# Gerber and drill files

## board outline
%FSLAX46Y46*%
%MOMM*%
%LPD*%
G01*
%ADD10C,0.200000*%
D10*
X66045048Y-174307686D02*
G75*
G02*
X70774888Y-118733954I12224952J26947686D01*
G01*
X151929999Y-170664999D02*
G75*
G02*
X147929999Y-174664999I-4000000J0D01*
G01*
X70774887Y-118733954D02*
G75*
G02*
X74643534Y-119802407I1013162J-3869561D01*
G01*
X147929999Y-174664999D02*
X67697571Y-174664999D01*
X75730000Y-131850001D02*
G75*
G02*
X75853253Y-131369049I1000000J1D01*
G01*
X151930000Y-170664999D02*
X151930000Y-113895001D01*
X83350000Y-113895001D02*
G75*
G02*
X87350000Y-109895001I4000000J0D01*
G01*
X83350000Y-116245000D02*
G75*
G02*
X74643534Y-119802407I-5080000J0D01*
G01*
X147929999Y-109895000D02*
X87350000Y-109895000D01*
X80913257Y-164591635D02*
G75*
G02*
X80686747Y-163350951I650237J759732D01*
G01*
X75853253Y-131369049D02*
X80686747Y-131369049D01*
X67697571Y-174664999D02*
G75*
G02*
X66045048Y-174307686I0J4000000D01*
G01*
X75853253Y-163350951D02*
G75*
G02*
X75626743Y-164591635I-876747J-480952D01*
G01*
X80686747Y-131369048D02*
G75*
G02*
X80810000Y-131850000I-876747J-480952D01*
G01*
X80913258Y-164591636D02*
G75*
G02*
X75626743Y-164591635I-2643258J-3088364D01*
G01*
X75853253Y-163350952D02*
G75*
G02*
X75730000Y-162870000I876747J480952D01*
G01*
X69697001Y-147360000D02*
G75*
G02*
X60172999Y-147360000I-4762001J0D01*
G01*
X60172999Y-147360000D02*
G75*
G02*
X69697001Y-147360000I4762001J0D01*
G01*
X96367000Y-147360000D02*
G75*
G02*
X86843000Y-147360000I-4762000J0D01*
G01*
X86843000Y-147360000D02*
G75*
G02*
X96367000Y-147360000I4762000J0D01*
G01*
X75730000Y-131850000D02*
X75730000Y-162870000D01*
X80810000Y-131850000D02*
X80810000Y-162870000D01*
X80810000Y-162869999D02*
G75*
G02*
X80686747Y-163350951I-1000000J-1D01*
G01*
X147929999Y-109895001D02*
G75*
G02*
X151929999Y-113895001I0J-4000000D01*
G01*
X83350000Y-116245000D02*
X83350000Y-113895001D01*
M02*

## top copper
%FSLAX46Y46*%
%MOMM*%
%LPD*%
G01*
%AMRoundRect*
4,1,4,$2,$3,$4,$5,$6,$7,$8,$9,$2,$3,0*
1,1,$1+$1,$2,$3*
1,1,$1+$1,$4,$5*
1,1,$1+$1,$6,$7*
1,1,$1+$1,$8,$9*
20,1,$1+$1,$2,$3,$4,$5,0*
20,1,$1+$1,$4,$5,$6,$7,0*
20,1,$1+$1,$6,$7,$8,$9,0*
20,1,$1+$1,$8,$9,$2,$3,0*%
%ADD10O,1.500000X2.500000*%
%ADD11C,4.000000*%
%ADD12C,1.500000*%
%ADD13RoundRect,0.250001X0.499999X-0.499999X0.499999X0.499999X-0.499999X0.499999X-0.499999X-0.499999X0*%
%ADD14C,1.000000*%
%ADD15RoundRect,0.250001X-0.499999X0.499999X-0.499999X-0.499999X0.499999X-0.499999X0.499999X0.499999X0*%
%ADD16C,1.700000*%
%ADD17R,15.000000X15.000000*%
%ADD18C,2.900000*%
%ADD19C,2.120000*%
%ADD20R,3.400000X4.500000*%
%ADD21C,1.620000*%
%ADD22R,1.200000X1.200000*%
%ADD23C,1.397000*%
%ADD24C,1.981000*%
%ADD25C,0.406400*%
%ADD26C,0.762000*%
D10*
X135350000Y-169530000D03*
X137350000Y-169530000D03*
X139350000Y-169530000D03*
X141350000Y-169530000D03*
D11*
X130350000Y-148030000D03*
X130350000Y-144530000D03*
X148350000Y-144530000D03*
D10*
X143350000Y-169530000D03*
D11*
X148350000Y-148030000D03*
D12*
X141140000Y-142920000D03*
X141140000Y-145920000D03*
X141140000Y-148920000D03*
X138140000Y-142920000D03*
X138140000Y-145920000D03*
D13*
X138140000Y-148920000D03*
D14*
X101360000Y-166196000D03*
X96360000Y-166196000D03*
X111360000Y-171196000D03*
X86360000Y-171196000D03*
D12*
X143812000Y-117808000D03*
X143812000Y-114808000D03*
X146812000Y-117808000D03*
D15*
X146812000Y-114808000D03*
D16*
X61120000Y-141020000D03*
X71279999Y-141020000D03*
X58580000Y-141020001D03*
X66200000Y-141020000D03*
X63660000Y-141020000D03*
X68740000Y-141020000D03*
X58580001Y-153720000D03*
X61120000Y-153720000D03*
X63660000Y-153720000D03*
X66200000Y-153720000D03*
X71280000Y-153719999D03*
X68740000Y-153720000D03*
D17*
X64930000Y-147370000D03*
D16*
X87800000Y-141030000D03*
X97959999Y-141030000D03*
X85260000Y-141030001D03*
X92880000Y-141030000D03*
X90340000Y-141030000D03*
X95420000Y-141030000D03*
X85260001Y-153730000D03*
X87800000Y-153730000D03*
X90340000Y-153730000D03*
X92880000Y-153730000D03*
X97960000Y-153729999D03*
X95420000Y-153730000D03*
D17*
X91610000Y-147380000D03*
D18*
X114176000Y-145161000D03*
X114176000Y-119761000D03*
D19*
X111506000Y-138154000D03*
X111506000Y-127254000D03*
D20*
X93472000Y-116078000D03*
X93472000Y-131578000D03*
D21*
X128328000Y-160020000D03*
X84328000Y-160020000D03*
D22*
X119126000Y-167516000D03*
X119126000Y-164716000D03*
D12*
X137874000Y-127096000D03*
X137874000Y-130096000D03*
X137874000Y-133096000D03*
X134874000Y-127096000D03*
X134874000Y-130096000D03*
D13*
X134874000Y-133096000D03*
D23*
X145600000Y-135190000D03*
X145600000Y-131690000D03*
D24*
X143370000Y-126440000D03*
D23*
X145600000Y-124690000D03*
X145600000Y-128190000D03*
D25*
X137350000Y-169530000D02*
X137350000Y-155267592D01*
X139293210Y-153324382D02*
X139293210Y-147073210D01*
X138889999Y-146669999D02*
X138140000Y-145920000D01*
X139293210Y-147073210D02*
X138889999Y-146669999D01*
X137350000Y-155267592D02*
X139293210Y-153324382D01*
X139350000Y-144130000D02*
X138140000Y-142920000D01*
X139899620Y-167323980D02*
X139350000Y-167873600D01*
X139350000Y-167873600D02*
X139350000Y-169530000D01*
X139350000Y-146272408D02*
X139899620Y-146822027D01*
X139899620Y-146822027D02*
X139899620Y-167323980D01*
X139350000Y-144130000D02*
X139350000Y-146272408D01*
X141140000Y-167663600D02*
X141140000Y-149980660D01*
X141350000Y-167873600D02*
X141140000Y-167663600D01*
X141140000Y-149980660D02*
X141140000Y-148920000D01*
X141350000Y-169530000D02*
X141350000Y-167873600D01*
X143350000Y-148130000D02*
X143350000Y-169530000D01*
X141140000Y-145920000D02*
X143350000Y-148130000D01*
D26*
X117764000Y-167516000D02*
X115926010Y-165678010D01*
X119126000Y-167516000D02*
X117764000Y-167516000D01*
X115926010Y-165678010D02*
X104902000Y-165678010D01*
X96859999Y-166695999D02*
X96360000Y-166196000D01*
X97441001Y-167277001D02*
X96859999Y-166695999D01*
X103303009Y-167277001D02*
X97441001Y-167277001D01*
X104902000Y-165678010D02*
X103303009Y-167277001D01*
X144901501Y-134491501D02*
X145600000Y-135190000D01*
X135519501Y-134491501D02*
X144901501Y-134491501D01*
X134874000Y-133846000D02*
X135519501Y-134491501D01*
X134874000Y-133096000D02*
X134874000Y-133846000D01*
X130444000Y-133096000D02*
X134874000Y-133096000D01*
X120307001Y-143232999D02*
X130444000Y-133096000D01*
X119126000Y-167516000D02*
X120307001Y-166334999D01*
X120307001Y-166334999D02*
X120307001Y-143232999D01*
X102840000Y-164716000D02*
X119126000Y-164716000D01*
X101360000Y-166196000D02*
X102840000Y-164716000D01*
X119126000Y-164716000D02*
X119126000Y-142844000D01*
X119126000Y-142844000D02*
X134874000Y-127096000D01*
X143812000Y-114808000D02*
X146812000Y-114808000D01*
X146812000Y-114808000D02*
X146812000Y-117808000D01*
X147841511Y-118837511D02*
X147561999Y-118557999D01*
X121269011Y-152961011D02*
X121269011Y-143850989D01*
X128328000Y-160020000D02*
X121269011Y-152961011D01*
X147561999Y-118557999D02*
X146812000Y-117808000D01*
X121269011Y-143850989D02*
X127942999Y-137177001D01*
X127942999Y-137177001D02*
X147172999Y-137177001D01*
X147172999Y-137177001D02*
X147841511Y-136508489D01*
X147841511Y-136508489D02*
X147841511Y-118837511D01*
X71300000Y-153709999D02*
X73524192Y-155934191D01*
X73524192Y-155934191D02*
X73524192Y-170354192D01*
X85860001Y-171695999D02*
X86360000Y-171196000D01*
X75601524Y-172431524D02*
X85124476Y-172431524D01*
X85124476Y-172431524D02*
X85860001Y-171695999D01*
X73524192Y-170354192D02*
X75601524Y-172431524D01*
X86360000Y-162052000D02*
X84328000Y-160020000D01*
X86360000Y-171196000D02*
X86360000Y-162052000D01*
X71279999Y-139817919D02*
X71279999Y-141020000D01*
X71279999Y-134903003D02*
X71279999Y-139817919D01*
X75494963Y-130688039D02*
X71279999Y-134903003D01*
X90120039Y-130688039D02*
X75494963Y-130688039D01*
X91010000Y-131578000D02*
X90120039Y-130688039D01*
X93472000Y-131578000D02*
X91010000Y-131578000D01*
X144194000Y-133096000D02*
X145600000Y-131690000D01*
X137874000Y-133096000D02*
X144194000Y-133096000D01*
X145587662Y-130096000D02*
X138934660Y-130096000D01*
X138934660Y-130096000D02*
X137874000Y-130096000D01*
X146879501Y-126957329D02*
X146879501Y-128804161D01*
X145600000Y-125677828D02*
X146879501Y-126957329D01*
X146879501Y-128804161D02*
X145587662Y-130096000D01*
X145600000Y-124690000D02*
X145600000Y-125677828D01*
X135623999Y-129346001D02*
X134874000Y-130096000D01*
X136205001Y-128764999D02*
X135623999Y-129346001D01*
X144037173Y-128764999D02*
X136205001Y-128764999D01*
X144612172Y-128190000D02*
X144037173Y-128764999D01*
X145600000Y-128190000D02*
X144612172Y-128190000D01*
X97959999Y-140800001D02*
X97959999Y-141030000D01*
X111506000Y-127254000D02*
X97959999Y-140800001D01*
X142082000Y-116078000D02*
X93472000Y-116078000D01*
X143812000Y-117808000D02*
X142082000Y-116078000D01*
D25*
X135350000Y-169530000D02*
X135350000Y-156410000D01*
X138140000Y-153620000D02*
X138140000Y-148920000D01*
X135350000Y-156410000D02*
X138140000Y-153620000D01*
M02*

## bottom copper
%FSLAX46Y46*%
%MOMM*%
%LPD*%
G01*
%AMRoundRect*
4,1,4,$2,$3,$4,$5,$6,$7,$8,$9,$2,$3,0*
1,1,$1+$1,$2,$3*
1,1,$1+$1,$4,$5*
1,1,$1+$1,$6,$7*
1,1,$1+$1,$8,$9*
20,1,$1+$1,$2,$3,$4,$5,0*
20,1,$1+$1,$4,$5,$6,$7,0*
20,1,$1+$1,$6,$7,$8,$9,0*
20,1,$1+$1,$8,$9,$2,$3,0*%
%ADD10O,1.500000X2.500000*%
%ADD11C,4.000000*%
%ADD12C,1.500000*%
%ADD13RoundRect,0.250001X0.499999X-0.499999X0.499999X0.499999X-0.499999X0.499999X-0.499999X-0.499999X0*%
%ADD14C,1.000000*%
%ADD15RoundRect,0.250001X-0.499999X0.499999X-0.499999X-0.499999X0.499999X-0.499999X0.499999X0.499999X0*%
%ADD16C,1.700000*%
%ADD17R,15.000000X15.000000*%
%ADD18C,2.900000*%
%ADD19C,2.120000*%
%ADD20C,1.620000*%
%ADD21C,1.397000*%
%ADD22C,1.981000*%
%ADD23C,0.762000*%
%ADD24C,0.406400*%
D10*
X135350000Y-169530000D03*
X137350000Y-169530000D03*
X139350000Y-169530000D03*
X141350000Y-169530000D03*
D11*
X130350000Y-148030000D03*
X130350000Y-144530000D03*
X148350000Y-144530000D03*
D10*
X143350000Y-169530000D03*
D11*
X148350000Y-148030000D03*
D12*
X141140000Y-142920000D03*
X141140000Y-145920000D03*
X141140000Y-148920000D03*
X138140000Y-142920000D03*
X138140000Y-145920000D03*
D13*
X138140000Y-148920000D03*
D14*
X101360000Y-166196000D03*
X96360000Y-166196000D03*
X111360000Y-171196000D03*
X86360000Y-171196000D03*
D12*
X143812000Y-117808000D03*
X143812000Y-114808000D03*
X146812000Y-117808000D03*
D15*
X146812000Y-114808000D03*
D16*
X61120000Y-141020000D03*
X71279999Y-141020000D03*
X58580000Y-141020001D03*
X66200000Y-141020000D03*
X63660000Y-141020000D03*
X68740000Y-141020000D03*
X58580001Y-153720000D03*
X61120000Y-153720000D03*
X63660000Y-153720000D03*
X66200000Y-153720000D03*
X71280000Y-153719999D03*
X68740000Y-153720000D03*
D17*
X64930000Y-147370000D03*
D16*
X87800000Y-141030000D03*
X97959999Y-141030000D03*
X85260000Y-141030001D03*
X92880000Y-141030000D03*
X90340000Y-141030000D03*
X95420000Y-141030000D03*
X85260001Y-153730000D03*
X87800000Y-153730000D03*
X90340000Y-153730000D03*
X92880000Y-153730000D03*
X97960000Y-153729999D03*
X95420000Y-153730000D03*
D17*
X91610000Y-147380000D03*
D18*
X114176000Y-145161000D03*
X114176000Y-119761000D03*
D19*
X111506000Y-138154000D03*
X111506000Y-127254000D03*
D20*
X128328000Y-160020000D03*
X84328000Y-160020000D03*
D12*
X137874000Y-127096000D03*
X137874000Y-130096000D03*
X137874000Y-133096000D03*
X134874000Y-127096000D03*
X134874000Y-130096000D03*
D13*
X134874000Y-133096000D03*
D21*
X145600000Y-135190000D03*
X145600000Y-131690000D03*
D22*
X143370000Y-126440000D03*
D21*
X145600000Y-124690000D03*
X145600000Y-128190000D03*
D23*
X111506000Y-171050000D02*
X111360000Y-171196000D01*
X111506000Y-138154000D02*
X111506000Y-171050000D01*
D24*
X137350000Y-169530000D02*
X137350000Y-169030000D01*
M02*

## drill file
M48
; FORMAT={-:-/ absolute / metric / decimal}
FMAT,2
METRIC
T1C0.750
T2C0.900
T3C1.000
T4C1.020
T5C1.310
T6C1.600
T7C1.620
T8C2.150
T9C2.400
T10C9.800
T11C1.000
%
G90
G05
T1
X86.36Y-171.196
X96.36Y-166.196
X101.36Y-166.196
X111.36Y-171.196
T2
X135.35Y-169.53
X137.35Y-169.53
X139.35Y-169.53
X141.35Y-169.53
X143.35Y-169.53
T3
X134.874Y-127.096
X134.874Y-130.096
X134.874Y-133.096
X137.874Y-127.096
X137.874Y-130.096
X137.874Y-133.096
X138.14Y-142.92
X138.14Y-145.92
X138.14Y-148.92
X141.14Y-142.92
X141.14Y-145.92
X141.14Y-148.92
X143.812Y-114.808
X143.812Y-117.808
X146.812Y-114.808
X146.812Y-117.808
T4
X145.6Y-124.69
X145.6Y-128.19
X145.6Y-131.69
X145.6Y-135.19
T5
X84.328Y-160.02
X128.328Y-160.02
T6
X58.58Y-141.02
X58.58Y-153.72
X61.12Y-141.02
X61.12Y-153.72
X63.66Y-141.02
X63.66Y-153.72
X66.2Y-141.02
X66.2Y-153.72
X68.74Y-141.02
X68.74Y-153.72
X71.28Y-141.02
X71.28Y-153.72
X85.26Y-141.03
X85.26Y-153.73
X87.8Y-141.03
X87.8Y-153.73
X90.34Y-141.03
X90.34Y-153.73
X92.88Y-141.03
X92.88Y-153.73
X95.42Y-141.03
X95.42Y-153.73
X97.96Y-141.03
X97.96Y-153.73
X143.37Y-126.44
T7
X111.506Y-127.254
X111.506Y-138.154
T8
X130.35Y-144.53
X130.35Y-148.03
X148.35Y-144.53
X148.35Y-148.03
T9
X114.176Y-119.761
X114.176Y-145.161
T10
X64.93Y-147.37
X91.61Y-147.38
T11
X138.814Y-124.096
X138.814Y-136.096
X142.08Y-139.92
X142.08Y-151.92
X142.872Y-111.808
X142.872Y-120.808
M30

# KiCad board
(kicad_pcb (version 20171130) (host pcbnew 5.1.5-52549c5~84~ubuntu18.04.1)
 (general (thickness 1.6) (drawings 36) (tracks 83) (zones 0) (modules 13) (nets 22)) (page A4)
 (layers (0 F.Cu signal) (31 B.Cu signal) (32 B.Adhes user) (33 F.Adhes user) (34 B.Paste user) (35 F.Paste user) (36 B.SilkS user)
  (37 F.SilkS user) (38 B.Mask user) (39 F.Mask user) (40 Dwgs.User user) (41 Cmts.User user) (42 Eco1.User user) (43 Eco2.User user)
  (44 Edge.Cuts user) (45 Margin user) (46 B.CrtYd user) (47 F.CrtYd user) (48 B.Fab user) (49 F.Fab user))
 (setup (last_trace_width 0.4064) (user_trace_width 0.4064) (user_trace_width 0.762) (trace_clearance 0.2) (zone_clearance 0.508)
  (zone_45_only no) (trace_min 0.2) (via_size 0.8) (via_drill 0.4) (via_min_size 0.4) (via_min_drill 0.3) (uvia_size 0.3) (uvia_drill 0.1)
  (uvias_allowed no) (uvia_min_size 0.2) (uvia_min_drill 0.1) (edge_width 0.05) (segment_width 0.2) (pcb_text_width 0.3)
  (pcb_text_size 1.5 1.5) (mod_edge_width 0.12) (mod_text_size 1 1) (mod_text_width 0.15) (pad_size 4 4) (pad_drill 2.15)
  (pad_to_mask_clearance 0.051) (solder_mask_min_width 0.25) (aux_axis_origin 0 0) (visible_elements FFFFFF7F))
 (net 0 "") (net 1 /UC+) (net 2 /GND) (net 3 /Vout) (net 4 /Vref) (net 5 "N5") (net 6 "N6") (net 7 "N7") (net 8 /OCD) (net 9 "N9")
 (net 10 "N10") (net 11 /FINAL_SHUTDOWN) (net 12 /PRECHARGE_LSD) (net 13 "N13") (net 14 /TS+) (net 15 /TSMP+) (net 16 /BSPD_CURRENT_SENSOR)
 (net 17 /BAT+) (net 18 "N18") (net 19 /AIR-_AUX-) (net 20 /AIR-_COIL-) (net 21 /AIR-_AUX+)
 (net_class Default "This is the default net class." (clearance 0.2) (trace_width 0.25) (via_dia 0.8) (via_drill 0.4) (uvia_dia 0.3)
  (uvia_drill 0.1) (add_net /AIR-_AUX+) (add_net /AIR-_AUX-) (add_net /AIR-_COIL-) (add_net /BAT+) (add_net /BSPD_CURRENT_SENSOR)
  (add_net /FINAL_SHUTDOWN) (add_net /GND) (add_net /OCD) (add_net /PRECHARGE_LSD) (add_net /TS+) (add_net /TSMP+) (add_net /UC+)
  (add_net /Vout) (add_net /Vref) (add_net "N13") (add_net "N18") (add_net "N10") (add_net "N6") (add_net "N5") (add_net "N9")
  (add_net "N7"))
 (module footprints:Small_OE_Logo (layer F.Cu) (at 68.47 130.89)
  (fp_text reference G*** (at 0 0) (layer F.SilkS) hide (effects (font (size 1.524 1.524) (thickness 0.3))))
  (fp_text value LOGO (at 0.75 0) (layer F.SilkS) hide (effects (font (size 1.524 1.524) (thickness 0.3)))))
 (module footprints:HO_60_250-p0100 (layer B.Cu) (at 130.35 144.53 270)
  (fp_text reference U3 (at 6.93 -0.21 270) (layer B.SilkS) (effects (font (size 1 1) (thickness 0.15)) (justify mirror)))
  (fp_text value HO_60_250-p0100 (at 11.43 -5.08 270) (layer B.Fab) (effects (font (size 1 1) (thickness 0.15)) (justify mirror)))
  (pad 1 thru_hole oval (at 25 -5 270) (size 2.5 1.5) (drill 0.9) (layers *.Cu *.Mask) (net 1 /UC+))
  (pad 2 thru_hole oval (at 25 -7 270) (size 2.5 1.5) (drill 0.9) (layers *.Cu *.Mask) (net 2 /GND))
  (pad 3 thru_hole oval (at 25 -9 270) (size 2.5 1.5) (drill 0.9) (layers *.Cu *.Mask) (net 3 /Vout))
  (pad 4 thru_hole oval (at 25 -11 270) (size 2.5 1.5) (drill 0.9) (layers *.Cu *.Mask) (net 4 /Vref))
  (pad 12 thru_hole circle (at 3.5 0 270) (size 4 4) (drill 2.15) (layers *.Cu *.Mask) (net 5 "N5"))
  (pad 11 thru_hole circle (at 0 0 270) (size 4 4) (drill 2.15) (layers *.Cu *.Mask) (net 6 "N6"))
  (pad 8 thru_hole circle (at 0 -18 270) (size 4 4) (drill 2.15) (layers *.Cu *.Mask) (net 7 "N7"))
  (pad 5 thru_hole oval (at 25 -13 270) (size 2.5 1.5) (drill 0.9) (layers *.Cu *.Mask) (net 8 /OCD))
  (pad 7 thru_hole circle (at 3.5 -18 270) (size 4 4) (drill 2.15) (layers *.Cu *.Mask) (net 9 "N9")))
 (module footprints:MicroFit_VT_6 (layer F.Cu) (at 138.14 148.92 90)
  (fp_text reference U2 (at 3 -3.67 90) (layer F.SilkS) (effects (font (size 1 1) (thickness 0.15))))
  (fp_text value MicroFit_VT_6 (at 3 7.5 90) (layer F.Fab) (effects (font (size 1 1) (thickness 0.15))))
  (pad 6 thru_hole circle (at 6 3 90) (size 1.5 1.5) (drill 1) (layers *.Cu *.Mask) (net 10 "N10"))
  (pad 5 thru_hole circle (at 3 3 90) (size 1.5 1.5) (drill 1) (layers *.Cu *.Mask) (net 8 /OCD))
  (pad 4 thru_hole circle (at 0 3 90) (size 1.5 1.5) (drill 1) (layers *.Cu *.Mask) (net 4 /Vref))
  (pad 3 thru_hole circle (at 6 0 90) (size 1.5 1.5) (drill 1) (layers *.Cu *.Mask) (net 3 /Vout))
  (pad 2 thru_hole circle (at 3 0 90) (size 1.5 1.5) (drill 1) (layers *.Cu *.Mask) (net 2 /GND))
  (pad 1 thru_hole roundrect (at 0 0 90) (size 1.5 1.5) (drill 1) (layers *.Cu *.Mask) (roundrect_rratio 0.166667) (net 1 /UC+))
  (pad "" np_thru_hole circle (at 9 3.94 90) (size 1 1) (drill 1) (layers *.Cu *.Mask))
  (pad "" np_thru_hole circle (at -3 3.94 90) (size 1 1) (drill 1) (layers *.Cu *.Mask)))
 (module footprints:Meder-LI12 (layer F.Cu) (at 86.36 171.196)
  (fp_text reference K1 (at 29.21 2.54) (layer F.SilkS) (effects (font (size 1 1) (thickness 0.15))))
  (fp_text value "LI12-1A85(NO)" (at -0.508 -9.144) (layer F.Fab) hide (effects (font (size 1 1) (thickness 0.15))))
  (pad 4 thru_hole circle (at 15 -5) (size 1 1) (drill 0.75) (layers *.Cu *.Mask) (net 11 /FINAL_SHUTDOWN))
  (pad 3 thru_hole circle (at 10 -5) (size 1 1) (drill 0.75) (layers *.Cu *.Mask) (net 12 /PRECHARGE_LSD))
  (pad 2 thru_hole circle (at 25 0) (size 1 1) (drill 0.75) (layers *.Cu *.Mask) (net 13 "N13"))
  (pad 1 thru_hole circle (at 0 0) (size 1 1) (drill 0.75) (layers *.Cu *.Mask) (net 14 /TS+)))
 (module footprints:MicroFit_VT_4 (layer F.Cu) (at 146.812 114.808 270)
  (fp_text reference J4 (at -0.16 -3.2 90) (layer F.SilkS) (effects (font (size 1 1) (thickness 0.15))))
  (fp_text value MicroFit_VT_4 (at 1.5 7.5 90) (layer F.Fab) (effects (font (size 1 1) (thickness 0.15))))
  (pad 4 thru_hole circle (at 3 3 270) (size 1.5 1.5) (drill 1) (layers *.Cu *.Mask) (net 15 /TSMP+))
  (pad 3 thru_hole circle (at 0 3 270) (size 1.5 1.5) (drill 1) (layers *.Cu *.Mask) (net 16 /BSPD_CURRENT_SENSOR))
  (pad 2 thru_hole circle (at 3 0 270) (size 1.5 1.5) (drill 1) (layers *.Cu *.Mask) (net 16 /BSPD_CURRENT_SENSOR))
  (pad 1 thru_hole roundrect (at 0 0 270) (size 1.5 1.5) (drill 1) (layers *.Cu *.Mask) (roundrect_rratio 0.166667)
   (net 16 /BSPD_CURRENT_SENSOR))
  (pad "" np_thru_hole circle (at 6 3.94 270) (size 1 1) (drill 1) (layers *.Cu *.Mask))
  (pad "" np_thru_hole circle (at -3 3.94 270) (size 1 1) (drill 1) (layers *.Cu *.Mask)))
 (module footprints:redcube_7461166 (layer F.Cu) (at 64.93 147.37)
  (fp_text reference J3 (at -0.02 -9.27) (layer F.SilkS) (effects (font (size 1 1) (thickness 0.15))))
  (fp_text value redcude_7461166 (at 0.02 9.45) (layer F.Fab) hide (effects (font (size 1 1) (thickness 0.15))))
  (pad 1 thru_hole circle (at -3.81 -6.35) (size 1.7 1.7) (drill 1.6) (layers *.Cu *.Mask) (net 14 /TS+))
  (pad 1 thru_hole circle (at 6.349999 -6.35) (size 1.7 1.7) (drill 1.6) (layers *.Cu *.Mask) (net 14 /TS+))
  (pad 1 thru_hole circle (at -6.35 -6.349999) (size 1.7 1.7) (drill 1.6) (layers *.Cu *.Mask) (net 14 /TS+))
  (pad 1 thru_hole circle (at 1.27 -6.35) (size 1.7 1.7) (drill 1.6) (layers *.Cu *.Mask) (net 14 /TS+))
  (pad 1 thru_hole circle (at -1.27 -6.35) (size 1.7 1.7) (drill 1.6) (layers *.Cu *.Mask) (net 14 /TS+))
  (pad 1 thru_hole circle (at 3.81 -6.35) (size 1.7 1.7) (drill 1.6) (layers *.Cu *.Mask) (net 14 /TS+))
  (pad 1 thru_hole circle (at -6.349999 6.35) (size 1.7 1.7) (drill 1.6) (layers *.Cu *.Mask) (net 14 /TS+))
  (pad 1 thru_hole circle (at -3.81 6.35) (size 1.7 1.7) (drill 1.6) (layers *.Cu *.Mask) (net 14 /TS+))
  (pad 1 thru_hole circle (at -1.27 6.35) (size 1.7 1.7) (drill 1.6) (layers *.Cu *.Mask) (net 14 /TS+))
  (pad 1 thru_hole circle (at 1.27 6.35) (size 1.7 1.7) (drill 1.6) (layers *.Cu *.Mask) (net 14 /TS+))
  (pad 1 thru_hole circle (at 6.35 6.349999) (size 1.7 1.7) (drill 1.6) (layers *.Cu *.Mask) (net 14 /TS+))
  (pad 1 thru_hole circle (at 3.81 6.35) (size 1.7 1.7) (drill 1.6) (layers *.Cu *.Mask) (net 14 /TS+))
  (pad 1 thru_hole rect (at 0 0) (size 15 15) (drill 9.8) (layers *.Cu *.Mask) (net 14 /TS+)))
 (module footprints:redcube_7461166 (layer F.Cu) (at 91.61 147.38)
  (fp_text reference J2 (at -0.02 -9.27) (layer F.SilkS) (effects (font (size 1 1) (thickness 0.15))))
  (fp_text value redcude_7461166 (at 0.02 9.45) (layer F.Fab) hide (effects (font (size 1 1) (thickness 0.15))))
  (pad 1 thru_hole circle (at -3.81 -6.35) (size 1.7 1.7) (drill 1.6) (layers *.Cu *.Mask) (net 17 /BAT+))
  (pad 1 thru_hole circle (at 6.349999 -6.35) (size 1.7 1.7) (drill 1.6) (layers *.Cu *.Mask) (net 17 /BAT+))
  (pad 1 thru_hole circle (at -6.35 -6.349999) (size 1.7 1.7) (drill 1.6) (layers *.Cu *.Mask) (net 17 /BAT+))
  (pad 1 thru_hole circle (at 1.27 -6.35) (size 1.7 1.7) (drill 1.6) (layers *.Cu *.Mask) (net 17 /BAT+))
  (pad 1 thru_hole circle (at -1.27 -6.35) (size 1.7 1.7) (drill 1.6) (layers *.Cu *.Mask) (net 17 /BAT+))
  (pad 1 thru_hole circle (at 3.81 -6.35) (size 1.7 1.7) (drill 1.6) (layers *.Cu *.Mask) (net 17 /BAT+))
  (pad 1 thru_hole circle (at -6.349999 6.35) (size 1.7 1.7) (drill 1.6) (layers *.Cu *.Mask) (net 17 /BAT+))
  (pad 1 thru_hole circle (at -3.81 6.35) (size 1.7 1.7) (drill 1.6) (layers *.Cu *.Mask) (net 17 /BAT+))
  (pad 1 thru_hole circle (at -1.27 6.35) (size 1.7 1.7) (drill 1.6) (layers *.Cu *.Mask) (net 17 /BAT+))
  (pad 1 thru_hole circle (at 1.27 6.35) (size 1.7 1.7) (drill 1.6) (layers *.Cu *.Mask) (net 17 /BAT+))
  (pad 1 thru_hole circle (at 6.35 6.349999) (size 1.7 1.7) (drill 1.6) (layers *.Cu *.Mask) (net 17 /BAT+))
  (pad 1 thru_hole circle (at 3.81 6.35) (size 1.7 1.7) (drill 1.6) (layers *.Cu *.Mask) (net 17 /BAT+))
  (pad 1 thru_hole rect (at 0 0) (size 15 15) (drill 9.8) (layers *.Cu *.Mask) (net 17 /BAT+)))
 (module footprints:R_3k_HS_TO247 (layer F.Cu) (at 111.506 127.254 270)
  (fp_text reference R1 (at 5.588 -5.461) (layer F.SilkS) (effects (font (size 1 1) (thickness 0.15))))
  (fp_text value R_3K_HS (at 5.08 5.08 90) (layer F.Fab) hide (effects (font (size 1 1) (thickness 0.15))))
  (pad 5 thru_hole circle (at 17.907 -2.67 270) (size 2.9 2.9) (drill 2.4) (layers *.Cu *.Mask))
  (pad 4 thru_hole circle (at -7.493 -2.67 270) (size 2.9 2.9) (drill 2.4) (layers *.Cu *.Mask))
  (pad 2 thru_hole circle (at 10.9 0 270) (size 2.12 2.12) (drill 1.62) (layers *.Cu *.Mask) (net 13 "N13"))
  (pad 1 thru_hole circle (at 0 0 270) (size 2.12 2.12) (drill 1.62) (layers *.Cu *.Mask) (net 17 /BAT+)))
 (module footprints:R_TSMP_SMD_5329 (layer F.Cu) (at 93.472 123.698 270)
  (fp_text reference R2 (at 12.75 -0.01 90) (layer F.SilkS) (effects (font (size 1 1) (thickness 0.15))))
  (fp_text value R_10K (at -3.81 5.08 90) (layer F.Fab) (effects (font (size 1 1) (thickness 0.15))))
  (pad 1 smd rect (at -7.62 0 270) (size 4.5 3.4) (layers F.Cu F.Paste F.Mask) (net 15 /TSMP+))
  (pad 2 smd rect (at 7.88 0 270) (size 4.5 3.4) (layers F.Cu F.Paste F.Mask) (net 14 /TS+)))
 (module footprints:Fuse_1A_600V (layer F.Cu) (at 84.328 160.02)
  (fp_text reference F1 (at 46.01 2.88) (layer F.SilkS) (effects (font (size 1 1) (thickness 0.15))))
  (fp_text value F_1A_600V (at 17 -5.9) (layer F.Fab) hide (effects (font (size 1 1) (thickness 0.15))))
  (pad 2 thru_hole circle (at 44 0) (size 1.62 1.62) (drill 1.31) (layers *.Cu *.Mask) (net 16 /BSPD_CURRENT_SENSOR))
  (pad 1 thru_hole circle (at 0 0) (size 1.62 1.62) (drill 1.31) (layers *.Cu *.Mask) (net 14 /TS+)))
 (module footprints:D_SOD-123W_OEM (layer F.Cu) (at 119.126 166.116 270)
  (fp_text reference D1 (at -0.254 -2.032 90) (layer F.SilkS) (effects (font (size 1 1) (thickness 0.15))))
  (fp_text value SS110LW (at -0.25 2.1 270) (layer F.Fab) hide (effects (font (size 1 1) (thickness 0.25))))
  (pad 2 smd rect (at 1.4 0 270) (size 1.2 1.2) (layers F.Cu F.Paste F.Mask) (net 12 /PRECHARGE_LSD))
  (pad 1 smd rect (at -1.4 0 270) (size 1.2 1.2) (layers F.Cu F.Paste F.Mask) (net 11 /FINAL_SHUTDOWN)))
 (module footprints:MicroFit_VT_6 (layer F.Cu) (at 134.874 133.096 90)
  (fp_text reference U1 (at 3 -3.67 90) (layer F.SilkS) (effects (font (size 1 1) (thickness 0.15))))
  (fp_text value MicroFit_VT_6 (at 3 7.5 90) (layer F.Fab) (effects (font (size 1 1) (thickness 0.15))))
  (pad 6 thru_hole circle (at 6 3 90) (size 1.5 1.5) (drill 1) (layers *.Cu *.Mask) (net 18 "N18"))
  (pad 5 thru_hole circle (at 3 3 90) (size 1.5 1.5) (drill 1) (layers *.Cu *.Mask) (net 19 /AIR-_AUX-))
  (pad 4 thru_hole circle (at 0 3 90) (size 1.5 1.5) (drill 1) (layers *.Cu *.Mask) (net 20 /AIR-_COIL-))
  (pad 3 thru_hole circle (at 6 0 90) (size 1.5 1.5) (drill 1) (layers *.Cu *.Mask) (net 11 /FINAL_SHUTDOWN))
  (pad 2 thru_hole circle (at 3 0 90) (size 1.5 1.5) (drill 1) (layers *.Cu *.Mask) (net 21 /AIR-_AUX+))
  (pad 1 thru_hole roundrect (at 0 0 90) (size 1.5 1.5) (drill 1) (layers *.Cu *.Mask) (roundrect_rratio 0.166667) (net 12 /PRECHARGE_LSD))
  (pad "" np_thru_hole circle (at 9 3.94 90) (size 1 1) (drill 1) (layers *.Cu *.Mask))
  (pad "" np_thru_hole circle (at -3 3.94 90) (size 1 1) (drill 1) (layers *.Cu *.Mask)))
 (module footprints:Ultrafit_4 (layer F.Cu) (at 145.6 129.94 180)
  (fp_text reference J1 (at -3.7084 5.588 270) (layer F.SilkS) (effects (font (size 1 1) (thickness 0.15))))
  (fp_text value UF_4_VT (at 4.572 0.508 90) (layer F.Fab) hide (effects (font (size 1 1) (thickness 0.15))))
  (pad 4 thru_hole circle (at 0 -5.25) (size 1.397 1.397) (drill 1.02) (layers *.Cu *.Mask) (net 12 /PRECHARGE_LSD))
  (pad 3 thru_hole circle (at 0 -1.75) (size 1.397 1.397) (drill 1.02) (layers *.Cu *.Mask) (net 20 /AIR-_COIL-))
  (pad "" thru_hole circle (at 2.23 3.5 180) (size 1.981 1.981) (drill 1.6) (layers *.Cu *.Mask))
  (pad 1 thru_hole circle (at 0 5.25 180) (size 1.397 1.397) (drill 1.02) (layers *.Cu *.Mask) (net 19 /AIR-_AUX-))
  (pad 2 thru_hole circle (at 0 1.75 180) (size 1.397 1.397) (drill 1.02) (layers *.Cu *.Mask) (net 21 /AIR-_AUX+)))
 (gr_arc (start 78.27 147.36) (end 70.774888 118.733954) (angle -140.9260442) (layer Edge.Cuts) (width 0.2))
 (gr_arc (start 147.929999 170.664999) (end 147.929999 174.664999) (angle -90) (layer Edge.Cuts) (width 0.2))
 (gr_arc (start 71.788049 122.603515) (end 74.643534 119.802407) (angle -60.22307557) (layer Edge.Cuts) (width 0.2))
 (gr_line (start 147.929999 174.664999) (end 67.697571 174.664999) (layer Edge.Cuts) (width 0.2))
 (gr_arc (start 76.73 131.85) (end 75.853253 131.369049) (angle -28.74758428) (layer Edge.Cuts) (width 0.2))
 (gr_line (start 151.93 170.664999) (end 151.93 113.895001) (layer Edge.Cuts) (width 0.2))
 (gr_arc (start 87.35 113.895001) (end 87.35 109.895001) (angle -90) (layer Edge.Cuts) (width 0.2))
 (gr_arc (start 78.27 116.245) (end 74.643534 119.802407) (angle -135.5507758) (layer Edge.Cuts) (width 0.2))
 (gr_line (start 147.929999 109.895) (end 87.35 109.895) (layer Edge.Cuts) (width 0.2))
 (gr_arc (start 81.563494 163.831903) (end 80.686747 163.350951) (angle -78.18815309) (layer Edge.Cuts) (width 0.2))
 (gr_line (start 75.853253 131.369049) (end 80.686747 131.369049) (layer Edge.Cuts) (width 0.2))
 (gr_arc (start 67.697571 170.664999) (end 66.045048 174.307686) (angle -24.40165601) (layer Edge.Cuts) (width 0.2))
 (gr_arc (start 74.976506 163.831903) (end 75.626743 164.591635) (angle -78.18815309) (layer Edge.Cuts) (width 0.2))
 (gr_arc (start 79.81 131.85) (end 80.81 131.85) (angle -28.74758428) (layer Edge.Cuts) (width 0.2))
 (gr_arc (start 78.27 167.68) (end 75.626743 164.591635) (angle -278.8811376) (layer Edge.Cuts) (width 0.2))
 (gr_arc (start 76.73 162.87) (end 75.73 162.87) (angle -28.74758428) (layer Edge.Cuts) (width 0.2))
 (gr_circle (center 64.935 147.36) (end 69.697001 147.36) (layer Edge.Cuts) (width 0.2))
 (gr_circle (center 91.605 147.36) (end 96.367 147.36) (layer Edge.Cuts) (width 0.2))
 (gr_line (start 75.73 131.85) (end 75.73 162.87) (layer Edge.Cuts) (width 0.2))
 (gr_line (start 80.81 131.85) (end 80.81 162.87) (layer Edge.Cuts) (width 0.2))
 (gr_arc (start 79.81 162.87) (end 80.686747 163.350951) (angle -28.74758428) (layer Edge.Cuts) (width 0.2))
 (gr_arc (start 147.929999 113.895001) (end 151.929999 113.895001) (angle -90) (layer Edge.Cuts) (width 0.2))
 (gr_line (start 83.35 116.245) (end 83.35 113.895001) (layer Edge.Cuts) (width 0.2))
 (segment (start 111.506 171.05) (end 111.36 171.196) (width 0.762) (layer B.Cu) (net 13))
 (segment (start 111.506 138.154) (end 111.506 171.05) (width 0.762) (layer B.Cu) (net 13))
 (segment (start 137.35 169.53) (end 137.35 169.03) (width 0.4064) (layer B.Cu) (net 2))
 (segment (start 137.35 169.53) (end 137.35 155.267592) (width 0.4064) (layer F.Cu) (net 2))
 (segment (start 139.29321 153.324382) (end 139.29321 147.07321) (width 0.4064) (layer F.Cu) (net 2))
 (segment (start 138.889999 146.669999) (end 138.14 145.92) (width 0.4064) (layer F.Cu) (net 2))
 (segment (start 139.29321 147.07321) (end 138.889999 146.669999) (width 0.4064) (layer F.Cu) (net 2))
 (segment (start 137.35 155.267592) (end 139.29321 153.324382) (width 0.4064) (layer F.Cu) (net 2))
 (segment (start 139.35 144.13) (end 138.14 142.92) (width 0.4064) (layer F.Cu) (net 3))
 (segment (start 139.89962 167.32398) (end 139.35 167.8736) (width 0.4064) (layer F.Cu) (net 3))
 (segment (start 139.35 167.8736) (end 139.35 169.53) (width 0.4064) (layer F.Cu) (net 3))
 (segment (start 139.35 146.272408) (end 139.89962 146.822027) (width 0.4064) (layer F.Cu) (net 3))
 (segment (start 139.89962 146.822027) (end 139.89962 167.32398) (width 0.4064) (layer F.Cu) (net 3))
 (segment (start 139.35 144.13) (end 139.35 146.272408) (width 0.4064) (layer F.Cu) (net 3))
 (segment (start 141.14 167.6636) (end 141.14 149.98066) (width 0.4064) (layer F.Cu) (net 4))
 (segment (start 141.35 167.8736) (end 141.14 167.6636) (width 0.4064) (layer F.Cu) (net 4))
 (segment (start 141.14 149.98066) (end 141.14 148.92) (width 0.4064) (layer F.Cu) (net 4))
 (segment (start 141.35 169.53) (end 141.35 167.8736) (width 0.4064) (layer F.Cu) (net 4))
 (segment (start 143.35 148.13) (end 143.35 169.53) (width 0.4064) (layer F.Cu) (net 8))
 (segment (start 141.14 145.92) (end 143.35 148.13) (width 0.4064) (layer F.Cu) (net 8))
 (segment (start 117.764 167.516) (end 115.92601 165.67801) (width 0.762) (layer F.Cu) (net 12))
 (segment (start 119.126 167.516) (end 117.764 167.516) (width 0.762) (layer F.Cu) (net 12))
 (segment (start 115.92601 165.67801) (end 104.902 165.67801) (width 0.762) (layer F.Cu) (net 12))
 (segment (start 96.859999 166.695999) (end 96.36 166.196) (width 0.762) (layer F.Cu) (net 12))
 (segment (start 97.441001 167.277001) (end 96.859999 166.695999) (width 0.762) (layer F.Cu) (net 12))
 (segment (start 103.303009 167.277001) (end 97.441001 167.277001) (width 0.762) (layer F.Cu) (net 12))
 (segment (start 104.902 165.67801) (end 103.303009 167.277001) (width 0.762) (layer F.Cu) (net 12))
 (segment (start 144.901501 134.491501) (end 145.6 135.19) (width 0.762) (layer F.Cu) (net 12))
 (segment (start 135.519501 134.491501) (end 144.901501 134.491501) (width 0.762) (layer F.Cu) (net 12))
 (segment (start 134.874 133.846) (end 135.519501 134.491501) (width 0.762) (layer F.Cu) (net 12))
 (segment (start 134.874 133.096) (end 134.874 133.846) (width 0.762) (layer F.Cu) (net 12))
 (segment (start 130.444 133.096) (end 134.874 133.096) (width 0.762) (layer F.Cu) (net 12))
 (segment (start 120.307001 143.232999) (end 130.444 133.096) (width 0.762) (layer F.Cu) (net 12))
 (segment (start 119.126 167.516) (end 120.307001 166.334999) (width 0.762) (layer F.Cu) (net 12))
 (segment (start 120.307001 166.334999) (end 120.307001 143.232999) (width 0.762) (layer F.Cu) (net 12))
 (segment (start 102.84 164.716) (end 119.126 164.716) (width 0.762) (layer F.Cu) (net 11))
 (segment (start 101.36 166.196) (end 102.84 164.716) (width 0.762) (layer F.Cu) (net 11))
 (segment (start 119.126 164.716) (end 119.126 142.844) (width 0.762) (layer F.Cu) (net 11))
 (segment (start 119.126 142.844) (end 134.874 127.096) (width 0.762) (layer F.Cu) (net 11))
 (segment (start 143.812 114.808) (end 146.812 114.808) (width 0.762) (layer F.Cu) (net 16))
 (segment (start 146.812 114.808) (end 146.812 117.808) (width 0.762) (layer F.Cu) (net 16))
 (segment (start 147.841511 118.837511) (end 147.561999 118.557999) (width 0.762) (layer F.Cu) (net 16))
 (segment (start 121.269011 152.961011) (end 121.269011 143.850989) (width 0.762) (layer F.Cu) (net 16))
 (segment (start 128.328 160.02) (end 121.269011 152.961011) (width 0.762) (layer F.Cu) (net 16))
 (segment (start 147.561999 118.557999) (end 146.812 117.808) (width 0.762) (layer F.Cu) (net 16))
 (segment (start 121.269011 143.850989) (end 127.942999 137.177001) (width 0.762) (layer F.Cu) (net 16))
 (segment (start 127.942999 137.177001) (end 147.172999 137.177001) (width 0.762) (layer F.Cu) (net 16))
 (segment (start 147.172999 137.177001) (end 147.841511 136.508489) (width 0.762) (layer F.Cu) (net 16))
 (segment (start 147.841511 136.508489) (end 147.841511 118.837511) (width 0.762) (layer F.Cu) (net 16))
 (segment (start 71.3 153.709999) (end 73.524192 155.934191) (width 0.762) (layer F.Cu) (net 14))
 (segment (start 73.524192 155.934191) (end 73.524192 170.354192) (width 0.762) (layer F.Cu) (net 14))
 (segment (start 85.860001 171.695999) (end 86.36 171.196) (width 0.762) (layer F.Cu) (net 14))
 (segment (start 75.601524 172.431524) (end 85.124476 172.431524) (width 0.762) (layer F.Cu) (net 14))
 (segment (start 85.124476 172.431524) (end 85.860001 171.695999) (width 0.762) (layer F.Cu) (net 14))
 (segment (start 73.524192 170.354192) (end 75.601524 172.431524) (width 0.762) (layer F.Cu) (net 14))
 (segment (start 86.36 162.052) (end 84.328 160.02) (width 0.762) (layer F.Cu) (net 14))
 (segment (start 86.36 171.196) (end 86.36 162.052) (width 0.762) (layer F.Cu) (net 14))
 (segment (start 71.279999 139.817919) (end 71.279999 141.02) (width 0.762) (layer F.Cu) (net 14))
 (segment (start 71.279999 134.903003) (end 71.279999 139.817919) (width 0.762) (layer F.Cu) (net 14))
 (segment (start 75.494963 130.688039) (end 71.279999 134.903003) (width 0.762) (layer F.Cu) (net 14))
 (segment (start 90.120039 130.688039) (end 75.494963 130.688039) (width 0.762) (layer F.Cu) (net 14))
 (segment (start 91.01 131.578) (end 90.120039 130.688039) (width 0.762) (layer F.Cu) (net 14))
 (segment (start 93.472 131.578) (end 91.01 131.578) (width 0.762) (layer F.Cu) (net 14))
 (segment (start 144.194 133.096) (end 145.6 131.69) (width 0.762) (layer F.Cu) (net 20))
 (segment (start 137.874 133.096) (end 144.194 133.096) (width 0.762) (layer F.Cu) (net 20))
 (segment (start 145.587662 130.096) (end 138.93466 130.096) (width 0.762) (layer F.Cu) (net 19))
 (segment (start 138.93466 130.096) (end 137.874 130.096) (width 0.762) (layer F.Cu) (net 19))
 (segment (start 146.879501 126.957329) (end 146.879501 128.804161) (width 0.762) (layer F.Cu) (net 19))
 (segment (start 145.6 125.677828) (end 146.879501 126.957329) (width 0.762) (layer F.Cu) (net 19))
 (segment (start 146.879501 128.804161) (end 145.587662 130.096) (width 0.762) (layer F.Cu) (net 19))
 (segment (start 145.6 124.69) (end 145.6 125.677828) (width 0.762) (layer F.Cu) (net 19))
 (segment (start 135.623999 129.346001) (end 134.874 130.096) (width 0.762) (layer F.Cu) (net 21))
 (segment (start 136.205001 128.764999) (end 135.623999 129.346001) (width 0.762) (layer F.Cu) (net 21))
 (segment (start 144.037173 128.764999) (end 136.205001 128.764999) (width 0.762) (layer F.Cu) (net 21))
 (segment (start 144.612172 128.19) (end 144.037173 128.764999) (width 0.762) (layer F.Cu) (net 21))
 (segment (start 145.6 128.19) (end 144.612172 128.19) (width 0.762) (layer F.Cu) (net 21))
 (segment (start 97.959999 140.800001) (end 97.959999 141.03) (width 0.762) (layer F.Cu) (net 17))
 (segment (start 111.506 127.254) (end 97.959999 140.800001) (width 0.762) (layer F.Cu) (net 17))
 (segment (start 142.082 116.078) (end 93.472 116.078) (width 0.762) (layer F.Cu) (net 15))
 (segment (start 143.812 117.808) (end 142.082 116.078) (width 0.762) (layer F.Cu) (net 15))
 (segment (start 135.35 169.53) (end 135.35 156.41) (width 0.4064) (layer F.Cu) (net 1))
 (segment (start 138.14 153.62) (end 138.14 148.92) (width 0.4064) (layer F.Cu) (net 1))
 (segment (start 135.35 156.41) (end 138.14 153.62) (width 0.4064) (layer F.Cu) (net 1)))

